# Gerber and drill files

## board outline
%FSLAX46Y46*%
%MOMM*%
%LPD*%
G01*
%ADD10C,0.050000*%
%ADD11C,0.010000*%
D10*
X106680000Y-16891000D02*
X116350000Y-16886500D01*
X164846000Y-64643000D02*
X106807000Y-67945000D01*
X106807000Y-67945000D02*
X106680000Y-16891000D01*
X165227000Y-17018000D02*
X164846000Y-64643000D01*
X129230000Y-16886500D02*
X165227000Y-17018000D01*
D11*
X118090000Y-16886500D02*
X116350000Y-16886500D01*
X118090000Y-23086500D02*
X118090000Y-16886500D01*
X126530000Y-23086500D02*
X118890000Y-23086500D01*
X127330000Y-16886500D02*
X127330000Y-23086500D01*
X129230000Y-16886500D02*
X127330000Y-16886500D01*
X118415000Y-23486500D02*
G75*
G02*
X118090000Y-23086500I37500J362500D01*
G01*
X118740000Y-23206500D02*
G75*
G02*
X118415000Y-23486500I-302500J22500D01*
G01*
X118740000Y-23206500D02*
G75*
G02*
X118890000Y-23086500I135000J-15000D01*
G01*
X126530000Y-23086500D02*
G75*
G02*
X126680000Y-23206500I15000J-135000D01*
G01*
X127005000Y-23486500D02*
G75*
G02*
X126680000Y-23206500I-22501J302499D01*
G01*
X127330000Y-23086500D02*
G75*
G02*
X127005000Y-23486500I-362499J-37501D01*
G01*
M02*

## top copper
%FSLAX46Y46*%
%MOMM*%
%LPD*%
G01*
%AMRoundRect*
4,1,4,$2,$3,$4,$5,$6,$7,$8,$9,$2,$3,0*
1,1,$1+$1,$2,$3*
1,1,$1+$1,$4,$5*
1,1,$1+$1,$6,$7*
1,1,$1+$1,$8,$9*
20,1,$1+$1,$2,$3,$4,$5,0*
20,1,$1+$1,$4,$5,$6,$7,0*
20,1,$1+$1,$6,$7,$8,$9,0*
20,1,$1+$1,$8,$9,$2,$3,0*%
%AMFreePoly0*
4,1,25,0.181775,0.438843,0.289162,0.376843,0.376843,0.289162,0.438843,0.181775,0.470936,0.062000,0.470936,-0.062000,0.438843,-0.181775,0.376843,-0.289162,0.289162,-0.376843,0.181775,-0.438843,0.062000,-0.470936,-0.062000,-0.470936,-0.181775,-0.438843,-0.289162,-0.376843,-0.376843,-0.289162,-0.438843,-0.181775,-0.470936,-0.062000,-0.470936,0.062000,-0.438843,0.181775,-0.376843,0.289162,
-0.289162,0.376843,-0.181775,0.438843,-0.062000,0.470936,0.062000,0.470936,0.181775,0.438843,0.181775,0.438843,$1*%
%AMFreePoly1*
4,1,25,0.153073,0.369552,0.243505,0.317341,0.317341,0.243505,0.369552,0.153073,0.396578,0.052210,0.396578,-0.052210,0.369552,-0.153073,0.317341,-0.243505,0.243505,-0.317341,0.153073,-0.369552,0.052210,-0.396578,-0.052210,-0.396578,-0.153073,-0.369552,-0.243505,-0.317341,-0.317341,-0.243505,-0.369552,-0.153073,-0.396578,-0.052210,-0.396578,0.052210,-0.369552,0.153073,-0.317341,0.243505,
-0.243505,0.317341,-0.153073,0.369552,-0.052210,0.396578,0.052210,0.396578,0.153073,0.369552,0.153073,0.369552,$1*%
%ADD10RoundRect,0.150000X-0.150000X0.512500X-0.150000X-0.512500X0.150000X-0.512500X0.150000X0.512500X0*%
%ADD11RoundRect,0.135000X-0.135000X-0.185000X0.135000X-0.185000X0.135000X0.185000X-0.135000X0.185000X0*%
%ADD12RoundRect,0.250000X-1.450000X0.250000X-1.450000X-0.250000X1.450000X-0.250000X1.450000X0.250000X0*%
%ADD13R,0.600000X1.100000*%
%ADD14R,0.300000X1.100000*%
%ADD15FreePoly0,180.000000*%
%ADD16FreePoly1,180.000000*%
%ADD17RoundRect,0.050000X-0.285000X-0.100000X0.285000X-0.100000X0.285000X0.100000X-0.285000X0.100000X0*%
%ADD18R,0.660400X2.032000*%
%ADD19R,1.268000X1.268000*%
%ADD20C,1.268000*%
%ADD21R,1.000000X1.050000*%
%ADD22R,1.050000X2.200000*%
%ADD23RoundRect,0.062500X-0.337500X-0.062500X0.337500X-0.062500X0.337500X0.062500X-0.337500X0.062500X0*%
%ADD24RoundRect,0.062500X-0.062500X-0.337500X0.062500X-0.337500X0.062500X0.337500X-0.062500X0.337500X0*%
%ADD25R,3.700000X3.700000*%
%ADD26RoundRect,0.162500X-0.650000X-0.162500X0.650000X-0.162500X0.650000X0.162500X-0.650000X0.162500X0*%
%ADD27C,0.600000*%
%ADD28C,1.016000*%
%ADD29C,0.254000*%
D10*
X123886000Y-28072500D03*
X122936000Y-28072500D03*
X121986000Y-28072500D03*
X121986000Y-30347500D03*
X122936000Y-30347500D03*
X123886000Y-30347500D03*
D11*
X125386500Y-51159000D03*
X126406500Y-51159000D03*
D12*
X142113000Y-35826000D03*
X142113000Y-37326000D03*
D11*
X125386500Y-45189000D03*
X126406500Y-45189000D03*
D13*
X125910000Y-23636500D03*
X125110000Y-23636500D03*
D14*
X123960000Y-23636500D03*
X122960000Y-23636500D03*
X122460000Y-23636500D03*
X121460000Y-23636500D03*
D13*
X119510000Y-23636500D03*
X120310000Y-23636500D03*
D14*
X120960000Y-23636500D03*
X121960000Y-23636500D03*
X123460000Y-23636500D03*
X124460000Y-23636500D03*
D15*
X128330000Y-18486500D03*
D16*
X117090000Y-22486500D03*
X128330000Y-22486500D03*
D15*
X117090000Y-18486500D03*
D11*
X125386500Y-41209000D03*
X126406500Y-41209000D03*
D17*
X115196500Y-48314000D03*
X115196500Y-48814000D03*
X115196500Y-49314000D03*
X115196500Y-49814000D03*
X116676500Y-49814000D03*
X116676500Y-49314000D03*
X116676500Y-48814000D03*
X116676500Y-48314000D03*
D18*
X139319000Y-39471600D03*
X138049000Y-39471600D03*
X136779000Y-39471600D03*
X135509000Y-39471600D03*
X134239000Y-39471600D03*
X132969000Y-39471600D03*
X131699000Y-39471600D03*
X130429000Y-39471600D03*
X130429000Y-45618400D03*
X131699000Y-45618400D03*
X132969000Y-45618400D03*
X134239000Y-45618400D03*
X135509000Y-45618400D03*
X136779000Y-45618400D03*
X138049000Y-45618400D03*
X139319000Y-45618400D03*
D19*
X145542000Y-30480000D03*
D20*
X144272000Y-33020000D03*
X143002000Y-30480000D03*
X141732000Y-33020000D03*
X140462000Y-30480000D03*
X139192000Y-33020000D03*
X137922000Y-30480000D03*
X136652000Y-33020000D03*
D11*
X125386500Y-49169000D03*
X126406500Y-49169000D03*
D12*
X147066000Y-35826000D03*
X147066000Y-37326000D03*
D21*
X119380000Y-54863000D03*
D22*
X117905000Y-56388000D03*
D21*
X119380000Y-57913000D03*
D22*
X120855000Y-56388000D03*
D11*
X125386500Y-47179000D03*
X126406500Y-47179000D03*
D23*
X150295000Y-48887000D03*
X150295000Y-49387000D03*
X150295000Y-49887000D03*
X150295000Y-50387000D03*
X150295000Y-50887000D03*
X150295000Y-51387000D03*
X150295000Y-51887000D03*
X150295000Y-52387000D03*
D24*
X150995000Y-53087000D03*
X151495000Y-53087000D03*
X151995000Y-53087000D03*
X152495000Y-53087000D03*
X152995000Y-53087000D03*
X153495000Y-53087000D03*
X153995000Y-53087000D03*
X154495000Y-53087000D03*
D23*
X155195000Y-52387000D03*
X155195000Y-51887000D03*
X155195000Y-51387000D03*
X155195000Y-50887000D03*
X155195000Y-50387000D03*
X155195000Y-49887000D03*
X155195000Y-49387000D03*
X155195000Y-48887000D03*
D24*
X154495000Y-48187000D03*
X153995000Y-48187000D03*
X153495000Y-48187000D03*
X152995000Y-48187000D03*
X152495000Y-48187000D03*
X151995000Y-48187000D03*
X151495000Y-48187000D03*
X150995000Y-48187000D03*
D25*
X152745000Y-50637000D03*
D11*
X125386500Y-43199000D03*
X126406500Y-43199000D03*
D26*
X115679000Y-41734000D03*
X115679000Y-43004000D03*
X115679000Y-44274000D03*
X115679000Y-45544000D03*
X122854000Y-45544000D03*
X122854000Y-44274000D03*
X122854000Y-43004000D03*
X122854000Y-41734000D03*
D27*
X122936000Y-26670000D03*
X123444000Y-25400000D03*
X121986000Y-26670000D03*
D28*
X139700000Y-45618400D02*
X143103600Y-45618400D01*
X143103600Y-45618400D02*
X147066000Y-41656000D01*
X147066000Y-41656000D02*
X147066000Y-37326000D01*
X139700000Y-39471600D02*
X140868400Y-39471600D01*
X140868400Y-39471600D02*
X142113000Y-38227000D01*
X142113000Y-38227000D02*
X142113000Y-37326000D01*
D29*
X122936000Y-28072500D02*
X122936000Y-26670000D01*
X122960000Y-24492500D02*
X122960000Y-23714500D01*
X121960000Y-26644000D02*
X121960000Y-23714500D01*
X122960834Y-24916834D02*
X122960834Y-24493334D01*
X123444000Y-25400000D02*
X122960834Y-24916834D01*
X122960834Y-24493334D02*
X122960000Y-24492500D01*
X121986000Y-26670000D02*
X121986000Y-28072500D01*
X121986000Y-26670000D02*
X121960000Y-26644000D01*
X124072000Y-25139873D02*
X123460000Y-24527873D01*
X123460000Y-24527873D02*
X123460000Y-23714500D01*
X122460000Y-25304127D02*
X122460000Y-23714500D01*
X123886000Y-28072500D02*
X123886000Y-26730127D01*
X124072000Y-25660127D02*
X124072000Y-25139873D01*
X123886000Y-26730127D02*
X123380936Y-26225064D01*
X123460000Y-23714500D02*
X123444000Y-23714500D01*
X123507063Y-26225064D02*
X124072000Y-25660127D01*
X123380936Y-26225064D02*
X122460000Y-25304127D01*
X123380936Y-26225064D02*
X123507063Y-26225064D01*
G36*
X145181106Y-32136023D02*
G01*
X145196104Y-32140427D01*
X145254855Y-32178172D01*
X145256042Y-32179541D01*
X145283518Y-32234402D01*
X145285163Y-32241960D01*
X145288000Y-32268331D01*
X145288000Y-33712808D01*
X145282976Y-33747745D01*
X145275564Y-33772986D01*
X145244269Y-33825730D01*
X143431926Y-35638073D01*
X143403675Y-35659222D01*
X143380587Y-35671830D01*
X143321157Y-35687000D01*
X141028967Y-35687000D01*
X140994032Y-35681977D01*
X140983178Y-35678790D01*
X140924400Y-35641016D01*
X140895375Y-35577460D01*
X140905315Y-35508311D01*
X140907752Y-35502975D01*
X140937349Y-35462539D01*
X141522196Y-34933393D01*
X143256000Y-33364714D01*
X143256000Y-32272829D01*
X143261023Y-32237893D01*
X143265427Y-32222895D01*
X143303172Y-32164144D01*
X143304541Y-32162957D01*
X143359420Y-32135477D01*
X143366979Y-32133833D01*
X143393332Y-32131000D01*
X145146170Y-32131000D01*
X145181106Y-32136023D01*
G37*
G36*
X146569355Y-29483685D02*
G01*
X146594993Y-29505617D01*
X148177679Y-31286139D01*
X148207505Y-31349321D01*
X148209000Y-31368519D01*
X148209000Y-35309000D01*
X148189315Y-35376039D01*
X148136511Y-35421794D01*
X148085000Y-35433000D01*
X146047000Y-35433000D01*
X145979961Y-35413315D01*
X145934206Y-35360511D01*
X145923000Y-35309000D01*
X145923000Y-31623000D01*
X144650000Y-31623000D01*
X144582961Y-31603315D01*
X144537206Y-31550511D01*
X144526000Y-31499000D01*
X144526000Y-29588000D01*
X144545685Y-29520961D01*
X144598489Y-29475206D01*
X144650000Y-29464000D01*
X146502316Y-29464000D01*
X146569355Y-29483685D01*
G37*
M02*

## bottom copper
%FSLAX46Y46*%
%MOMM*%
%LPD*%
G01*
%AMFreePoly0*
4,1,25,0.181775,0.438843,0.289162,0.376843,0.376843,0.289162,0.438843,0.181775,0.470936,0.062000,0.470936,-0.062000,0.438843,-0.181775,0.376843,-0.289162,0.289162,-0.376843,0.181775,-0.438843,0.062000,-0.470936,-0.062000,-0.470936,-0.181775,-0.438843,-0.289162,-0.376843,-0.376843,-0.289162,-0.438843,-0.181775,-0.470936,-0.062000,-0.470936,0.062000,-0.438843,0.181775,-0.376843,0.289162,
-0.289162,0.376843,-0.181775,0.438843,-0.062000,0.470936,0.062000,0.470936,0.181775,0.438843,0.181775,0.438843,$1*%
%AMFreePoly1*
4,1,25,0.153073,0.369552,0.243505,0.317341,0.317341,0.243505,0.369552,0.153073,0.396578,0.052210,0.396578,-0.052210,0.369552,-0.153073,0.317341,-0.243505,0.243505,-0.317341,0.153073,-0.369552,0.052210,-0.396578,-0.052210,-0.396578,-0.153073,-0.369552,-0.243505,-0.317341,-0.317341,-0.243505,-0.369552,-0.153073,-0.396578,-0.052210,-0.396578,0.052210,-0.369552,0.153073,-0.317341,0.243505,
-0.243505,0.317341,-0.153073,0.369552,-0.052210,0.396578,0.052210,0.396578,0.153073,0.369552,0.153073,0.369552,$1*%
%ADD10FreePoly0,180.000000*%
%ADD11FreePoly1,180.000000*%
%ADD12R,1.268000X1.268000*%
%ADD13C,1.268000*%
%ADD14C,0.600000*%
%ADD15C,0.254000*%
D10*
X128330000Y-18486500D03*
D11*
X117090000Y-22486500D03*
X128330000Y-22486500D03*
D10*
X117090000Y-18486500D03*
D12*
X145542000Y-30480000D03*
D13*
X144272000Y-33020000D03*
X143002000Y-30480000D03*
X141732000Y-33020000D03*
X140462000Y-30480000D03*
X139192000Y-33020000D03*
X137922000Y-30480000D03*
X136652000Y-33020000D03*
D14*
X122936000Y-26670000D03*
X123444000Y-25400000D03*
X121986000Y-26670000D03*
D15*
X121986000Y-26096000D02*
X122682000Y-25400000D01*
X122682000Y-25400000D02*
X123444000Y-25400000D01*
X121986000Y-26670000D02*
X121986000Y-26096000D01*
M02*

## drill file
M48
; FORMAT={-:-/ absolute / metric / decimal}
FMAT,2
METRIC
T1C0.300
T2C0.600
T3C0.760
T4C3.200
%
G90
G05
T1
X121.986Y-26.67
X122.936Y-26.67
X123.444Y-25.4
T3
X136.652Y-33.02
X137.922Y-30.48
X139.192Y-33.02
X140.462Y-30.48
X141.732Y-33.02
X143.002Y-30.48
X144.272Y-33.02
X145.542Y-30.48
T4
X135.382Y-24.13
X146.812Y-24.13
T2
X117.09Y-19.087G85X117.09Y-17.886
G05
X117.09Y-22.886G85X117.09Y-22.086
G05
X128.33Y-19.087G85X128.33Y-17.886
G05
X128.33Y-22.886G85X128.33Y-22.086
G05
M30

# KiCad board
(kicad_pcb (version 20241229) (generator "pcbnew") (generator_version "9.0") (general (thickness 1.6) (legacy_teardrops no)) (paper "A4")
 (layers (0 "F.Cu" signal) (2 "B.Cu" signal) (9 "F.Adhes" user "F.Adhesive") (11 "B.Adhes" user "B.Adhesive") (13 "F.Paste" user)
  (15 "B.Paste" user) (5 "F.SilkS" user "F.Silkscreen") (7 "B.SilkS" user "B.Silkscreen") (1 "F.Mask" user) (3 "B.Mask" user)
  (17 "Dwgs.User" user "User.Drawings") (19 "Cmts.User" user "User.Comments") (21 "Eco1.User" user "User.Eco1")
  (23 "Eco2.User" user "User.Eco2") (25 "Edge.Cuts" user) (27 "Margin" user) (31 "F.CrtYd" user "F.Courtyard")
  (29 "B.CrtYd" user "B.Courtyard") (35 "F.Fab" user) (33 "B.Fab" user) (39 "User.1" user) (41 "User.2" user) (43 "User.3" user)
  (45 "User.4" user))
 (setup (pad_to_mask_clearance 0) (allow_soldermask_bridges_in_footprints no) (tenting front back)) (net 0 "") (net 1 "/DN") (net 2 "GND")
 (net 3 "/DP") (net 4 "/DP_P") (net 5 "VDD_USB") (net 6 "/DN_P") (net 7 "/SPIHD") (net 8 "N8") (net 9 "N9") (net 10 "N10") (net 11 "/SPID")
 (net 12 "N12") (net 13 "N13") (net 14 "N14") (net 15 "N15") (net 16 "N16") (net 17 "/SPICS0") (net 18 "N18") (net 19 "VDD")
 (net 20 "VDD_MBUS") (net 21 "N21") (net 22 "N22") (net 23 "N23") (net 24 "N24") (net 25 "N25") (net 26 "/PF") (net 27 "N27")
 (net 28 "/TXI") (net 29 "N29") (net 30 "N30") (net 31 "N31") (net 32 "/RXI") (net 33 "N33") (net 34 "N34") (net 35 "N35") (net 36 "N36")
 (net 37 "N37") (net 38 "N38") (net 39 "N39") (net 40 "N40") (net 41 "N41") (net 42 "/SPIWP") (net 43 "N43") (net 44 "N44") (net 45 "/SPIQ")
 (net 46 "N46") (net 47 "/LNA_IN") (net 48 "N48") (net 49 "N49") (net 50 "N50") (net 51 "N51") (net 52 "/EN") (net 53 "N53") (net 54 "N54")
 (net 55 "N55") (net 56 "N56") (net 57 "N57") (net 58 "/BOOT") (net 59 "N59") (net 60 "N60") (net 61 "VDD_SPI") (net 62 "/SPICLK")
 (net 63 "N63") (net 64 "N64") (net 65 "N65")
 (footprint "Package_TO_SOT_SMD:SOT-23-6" (layer "F.Cu") (at 122.936 29.21 -90)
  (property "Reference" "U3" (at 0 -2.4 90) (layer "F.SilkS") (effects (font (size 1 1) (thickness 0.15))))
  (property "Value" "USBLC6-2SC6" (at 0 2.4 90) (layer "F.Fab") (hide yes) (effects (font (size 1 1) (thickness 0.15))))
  (pad "1" smd roundrect (at -1.1375 -0.95 270) (size 1.325 0.6) (layers "F.Cu" "F.Mask" "F.Paste") (roundrect_rratio 0.25) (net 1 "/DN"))
  (pad "2" smd roundrect (at -1.1375 0 270) (size 1.325 0.6) (layers "F.Cu" "F.Mask" "F.Paste") (roundrect_rratio 0.25) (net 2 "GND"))
  (pad "3" smd roundrect (at -1.1375 0.95 270) (size 1.325 0.6) (layers "F.Cu" "F.Mask" "F.Paste") (roundrect_rratio 0.25) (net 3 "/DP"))
  (pad "4" smd roundrect (at 1.1375 0.95 270) (size 1.325 0.6) (layers "F.Cu" "F.Mask" "F.Paste") (roundrect_rratio 0.25) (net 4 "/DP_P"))
  (pad "5" smd roundrect (at 1.1375 0 270) (size 1.325 0.6) (layers "F.Cu" "F.Mask" "F.Paste") (roundrect_rratio 0.25) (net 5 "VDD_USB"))
  (pad "6" smd roundrect (at 1.1375 -0.95 270) (size 1.325 0.6) (layers "F.Cu" "F.Mask" "F.Paste") (roundrect_rratio 0.25) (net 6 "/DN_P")))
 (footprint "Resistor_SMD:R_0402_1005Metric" (layer "F.Cu") (at 125.8965 51.159)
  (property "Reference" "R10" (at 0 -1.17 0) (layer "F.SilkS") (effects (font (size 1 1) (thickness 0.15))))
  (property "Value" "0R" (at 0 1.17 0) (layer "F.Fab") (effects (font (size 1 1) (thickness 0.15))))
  (pad "1" smd roundrect (at -0.51 0) (size 0.54 0.64) (layers "F.Cu" "F.Mask" "F.Paste") (roundrect_rratio 0.25) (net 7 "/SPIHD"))
  (pad "2" smd roundrect (at 0.51 0) (size 0.54 0.64) (layers "F.Cu" "F.Mask" "F.Paste") (roundrect_rratio 0.25) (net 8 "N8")))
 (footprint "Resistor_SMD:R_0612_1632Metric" (layer "F.Cu") (at 142.113 36.576 -90)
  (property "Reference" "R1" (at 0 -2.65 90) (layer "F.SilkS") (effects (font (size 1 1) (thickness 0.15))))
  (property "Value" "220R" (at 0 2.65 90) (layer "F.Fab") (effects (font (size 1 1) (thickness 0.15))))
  (pad "1" smd roundrect (at -0.75 0 270) (size 1 3.4) (layers "F.Cu" "F.Mask" "F.Paste") (roundrect_rratio 0.25) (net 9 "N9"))
  (pad "2" smd roundrect (at 0.75 0 270) (size 1 3.4) (layers "F.Cu" "F.Mask" "F.Paste") (roundrect_rratio 0.25) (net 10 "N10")))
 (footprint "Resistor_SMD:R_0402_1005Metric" (layer "F.Cu") (at 125.8965 45.189)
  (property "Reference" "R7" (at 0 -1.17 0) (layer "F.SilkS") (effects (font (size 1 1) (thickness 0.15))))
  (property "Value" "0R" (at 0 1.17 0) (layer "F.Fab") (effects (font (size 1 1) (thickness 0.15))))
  (pad "1" smd roundrect (at -0.51 0) (size 0.54 0.64) (layers "F.Cu" "F.Mask" "F.Paste") (roundrect_rratio 0.25) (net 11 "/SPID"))
  (pad "2" smd roundrect (at 0.51 0) (size 0.54 0.64) (layers "F.Cu" "F.Mask" "F.Paste") (roundrect_rratio 0.25) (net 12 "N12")))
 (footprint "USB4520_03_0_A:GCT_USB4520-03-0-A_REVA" (layer "F.Cu") (at 122.71 18.4865 180)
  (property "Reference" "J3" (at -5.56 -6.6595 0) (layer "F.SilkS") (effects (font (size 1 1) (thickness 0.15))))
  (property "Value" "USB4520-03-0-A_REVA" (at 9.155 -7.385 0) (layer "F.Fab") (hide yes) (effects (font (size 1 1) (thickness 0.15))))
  (fp_line (start 4.62 1.6) (end 6.36 1.6) (stroke (width 0.01) (type solid)) (layer "Edge.Cuts"))
  (fp_line (start 4.62 -4.6) (end 4.62 1.6) (stroke (width 0.01) (type solid)) (layer "Edge.Cuts"))
  (fp_line (start -3.82 -4.6) (end 3.82 -4.6) (stroke (width 0.01) (type solid)) (layer "Edge.Cuts"))
  (fp_line (start -4.62 1.6) (end -4.62 -4.6) (stroke (width 0.01) (type solid)) (layer "Edge.Cuts"))
  (fp_line (start -6.52 1.6) (end -4.62 1.6) (stroke (width 0.01) (type solid)) (layer "Edge.Cuts"))
  (fp_arc (start 4.295 -5) (mid 4.540343 -4.86731) (end 4.62 -4.6) (stroke (width 0.01) (type solid)) (layer "Edge.Cuts"))
  (fp_arc (start 3.97 -4.72) (mid 4.07451 -4.92731) (end 4.295 -5) (stroke (width 0.01) (type solid)) (layer "Edge.Cuts"))
  (fp_arc (start 3.97 -4.72) (mid 3.919853 -4.628934) (end 3.82 -4.6) (stroke (width 0.01) (type solid)) (layer "Edge.Cuts"))
  (fp_arc (start -3.82 -4.6) (mid -3.919853 -4.628934) (end -3.97 -4.72) (stroke (width 0.01) (type solid)) (layer "Edge.Cuts"))
  (fp_arc (start -4.295 -5) (mid -4.07451 -4.92731) (end -3.97 -4.72) (stroke (width 0.01) (type solid)) (layer "Edge.Cuts"))
  (fp_arc (start -4.62 -4.6) (mid -4.540343 -4.86731) (end -4.295 -5) (stroke (width 0.01) (type solid)) (layer "Edge.Cuts"))
  (pad "A1_B12" smd rect (at -3.2 -5.15 180) (size 0.6 1.1) (layers "F.Cu" "F.Mask" "F.Paste") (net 2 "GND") (solder_mask_margin 0.102))
  (pad "A4_B9" smd rect (at -2.4 -5.15 180) (size 0.6 1.1) (layers "F.Cu" "F.Mask" "F.Paste") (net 5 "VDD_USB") (solder_mask_margin 0.102))
  (pad "A5" smd rect (at -1.25 -5.15 180) (size 0.3 1.1) (layers "F.Cu" "F.Mask" "F.Paste") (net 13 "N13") (solder_mask_margin 0.102))
  (pad "A6" smd rect (at -0.25 -5.15 180) (size 0.3 1.1) (layers "F.Cu" "F.Mask" "F.Paste") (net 3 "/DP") (solder_mask_margin 0.102))
  (pad "A7" smd rect (at 0.25 -5.15 180) (size 0.3 1.1) (layers "F.Cu" "F.Mask" "F.Paste") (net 1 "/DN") (solder_mask_margin 0.102))
  (pad "A8" smd rect (at 1.25 -5.15 180) (size 0.3 1.1) (layers "F.Cu" "F.Mask" "F.Paste") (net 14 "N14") (solder_mask_margin 0.102))
  (pad "B1_A12" smd rect (at 3.2 -5.15 180) (size 0.6 1.1) (layers "F.Cu" "F.Mask" "F.Paste") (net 2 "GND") (solder_mask_margin 0.102))
  (pad "B4_A9" smd rect (at 2.4 -5.15 180) (size 0.6 1.1) (layers "F.Cu" "F.Mask" "F.Paste") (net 5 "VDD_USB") (solder_mask_margin 0.102))
  (pad "B5" smd rect (at 1.75 -5.15 180) (size 0.3 1.1) (layers "F.Cu" "F.Mask" "F.Paste") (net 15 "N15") (solder_mask_margin 0.102))
  (pad "B6" smd rect (at 0.75 -5.15 180) (size 0.3 1.1) (layers "F.Cu" "F.Mask" "F.Paste") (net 3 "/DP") (solder_mask_margin 0.102))
  (pad "B7" smd rect (at -0.75 -5.15 180) (size 0.3 1.1) (layers "F.Cu" "F.Mask" "F.Paste") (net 1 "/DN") (solder_mask_margin 0.102))
  (pad "B8" smd rect (at -1.75 -5.15 180) (size 0.3 1.1) (layers "F.Cu" "F.Mask" "F.Paste") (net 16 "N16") (solder_mask_margin 0.102))
  (pad "S1" thru_hole custom (at -5.62 0 180) (size 0.95 1.9) (drill oval 0.6 1.8) (layers "*.Cu") (remove_unused_layers no) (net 2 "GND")
   (thermal_bridge_angle 90) (options (clearance outline) (anchor circle)) (primitives))
  (pad "S2" thru_hole custom (at 5.62 -4 180) (size 0.8 1.6) (drill oval 0.6 1.4) (layers "*.Cu") (remove_unused_layers no) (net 2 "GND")
   (thermal_bridge_angle 90) (options (clearance outline) (anchor circle)) (primitives))
  (pad "S3" thru_hole custom (at -5.62 -4 180) (size 0.8 1.6) (drill oval 0.6 1.4) (layers "*.Cu") (remove_unused_layers no) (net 2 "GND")
   (thermal_bridge_angle 90) (options (clearance outline) (anchor circle)) (primitives))
  (pad "S4" thru_hole custom (at 5.62 0 180) (size 0.95 1.9) (drill oval 0.6 1.8) (layers "*.Cu") (remove_unused_layers no) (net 2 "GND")
   (thermal_bridge_angle 90) (options (clearance outline) (anchor circle)) (primitives)))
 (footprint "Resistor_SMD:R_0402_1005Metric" (layer "F.Cu") (at 125.8965 41.209)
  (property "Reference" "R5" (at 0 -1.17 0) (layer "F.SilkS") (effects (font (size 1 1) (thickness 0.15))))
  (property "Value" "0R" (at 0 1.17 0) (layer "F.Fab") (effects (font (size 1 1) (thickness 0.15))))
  (pad "1" smd roundrect (at -0.51 0) (size 0.54 0.64) (layers "F.Cu" "F.Mask" "F.Paste") (roundrect_rratio 0.25) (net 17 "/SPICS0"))
  (pad "2" smd roundrect (at 0.51 0) (size 0.54 0.64) (layers "F.Cu" "F.Mask" "F.Paste") (roundrect_rratio 0.25) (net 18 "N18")))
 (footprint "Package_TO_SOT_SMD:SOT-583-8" (layer "F.Cu") (at 115.9365 49.064)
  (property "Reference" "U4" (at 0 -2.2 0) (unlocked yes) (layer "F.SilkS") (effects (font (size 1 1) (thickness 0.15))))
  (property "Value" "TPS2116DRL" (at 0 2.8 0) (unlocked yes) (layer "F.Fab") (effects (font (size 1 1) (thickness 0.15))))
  (pad "1" smd roundrect (at -0.74 -0.75) (size 0.67 0.3) (layers "F.Cu" "F.Mask" "F.Paste") (roundrect_rratio 0.1666666667) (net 2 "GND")
   (thermal_bridge_angle 45))
  (pad "2" smd roundrect (at -0.74 -0.25) (size 0.67 0.3) (layers "F.Cu" "F.Mask" "F.Paste") (roundrect_rratio 0.1666666667) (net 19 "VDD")
   (thermal_bridge_angle 45))
  (pad "3" smd roundrect (at -0.74 0.25) (size 0.67 0.3) (layers "F.Cu" "F.Mask" "F.Paste") (roundrect_rratio 0.1666666667)
   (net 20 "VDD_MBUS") (thermal_bridge_angle 45))
  (pad "4" smd roundrect (at -0.74 0.75) (size 0.67 0.3) (layers "F.Cu" "F.Mask" "F.Paste") (roundrect_rratio 0.1666666667) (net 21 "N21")
   (thermal_bridge_angle 45))
  (pad "5" smd roundrect (at 0.74 0.75) (size 0.67 0.3) (layers "F.Cu" "F.Mask" "F.Paste") (roundrect_rratio 0.1666666667)
   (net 20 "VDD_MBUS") (thermal_bridge_angle 45))
  (pad "6" smd roundrect (at 0.74 0.25) (size 0.67 0.3) (layers "F.Cu" "F.Mask" "F.Paste") (roundrect_rratio 0.1666666667) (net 5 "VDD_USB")
   (thermal_bridge_angle 45))
  (pad "7" smd roundrect (at 0.74 -0.25) (size 0.67 0.3) (layers "F.Cu" "F.Mask" "F.Paste") (roundrect_rratio 0.1666666667) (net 19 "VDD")
   (thermal_bridge_angle 45))
  (pad "8" smd roundrect (at 0.74 -0.75) (size 0.67 0.3) (layers "F.Cu" "F.Mask" "F.Paste") (roundrect_rratio 0.1666666667) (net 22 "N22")
   (thermal_bridge_angle 45)))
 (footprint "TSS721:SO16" (layer "F.Cu") (at 134.874 42.545 180)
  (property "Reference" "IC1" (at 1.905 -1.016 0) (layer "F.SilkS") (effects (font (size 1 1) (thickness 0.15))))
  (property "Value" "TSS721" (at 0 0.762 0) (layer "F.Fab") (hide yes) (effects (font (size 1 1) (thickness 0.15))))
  (pad "1" smd rect (at -4.445 3.0734 180) (size 0.6604 2.032) (layers "F.Cu" "F.Mask" "F.Paste") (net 10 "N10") (solder_mask_margin 0.102))
  (pad "2" smd rect (at -3.175 3.0734 180) (size 0.6604 2.032) (layers "F.Cu" "F.Mask" "F.Paste") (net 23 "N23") (solder_mask_margin 0.102))
  (pad "3" smd rect (at -1.905 3.0734 180) (size 0.6604 2.032) (layers "F.Cu" "F.Mask" "F.Paste") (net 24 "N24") (solder_mask_margin 0.102))
  (pad "4" smd rect (at -0.635 3.0734 180) (size 0.6604 2.032) (layers "F.Cu" "F.Mask" "F.Paste") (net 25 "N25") (solder_mask_margin 0.102))
  (pad "5" smd rect (at 0.635 3.0734 180) (size 0.6604 2.032) (layers "F.Cu" "F.Mask" "F.Paste") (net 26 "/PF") (solder_mask_margin 0.102))
  (pad "6" smd rect (at 1.905 3.0734 180) (size 0.6604 2.032) (layers "F.Cu" "F.Mask" "F.Paste") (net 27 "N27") (solder_mask_margin 0.102))
  (pad "7" smd rect (at 3.175 3.0734 180) (size 0.6604 2.032) (layers "F.Cu" "F.Mask" "F.Paste") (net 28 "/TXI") (solder_mask_margin 0.102))
  (pad "8" smd rect (at 4.445 3.0734 180) (size 0.6604 2.032) (layers "F.Cu" "F.Mask" "F.Paste") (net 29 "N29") (solder_mask_margin 0.102))
  (pad "9" smd rect (at 4.445 -3.0734 180) (size 0.6604 2.032) (layers "F.Cu" "F.Mask" "F.Paste") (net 20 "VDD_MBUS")
   (solder_mask_margin 0.102))
  (pad "10" smd rect (at 3.175 -3.0734 180) (size 0.6604 2.032) (layers "F.Cu" "F.Mask" "F.Paste") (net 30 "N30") (solder_mask_margin 0.102))
  (pad "11" smd rect (at 1.905 -3.0734 180) (size 0.6604 2.032) (layers "F.Cu" "F.Mask" "F.Paste") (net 20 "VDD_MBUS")
   (solder_mask_margin 0.102))
  (pad "12" smd rect (at 0.635 -3.0734 180) (size 0.6604 2.032) (layers "F.Cu" "F.Mask" "F.Paste") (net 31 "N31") (solder_mask_margin 0.102))
  (pad "13" smd rect (at -0.635 -3.0734 180) (size 0.6604 2.032) (layers "F.Cu" "F.Mask" "F.Paste") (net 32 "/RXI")
   (solder_mask_margin 0.102))
  (pad "14" smd rect (at -1.905 -3.0734 180) (size 0.6604 2.032) (layers "F.Cu" "F.Mask" "F.Paste") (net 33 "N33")
   (solder_mask_margin 0.102))
  (pad "15" smd rect (at -3.175 -3.0734 180) (size 0.6604 2.032) (layers "F.Cu" "F.Mask" "F.Paste") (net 2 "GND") (solder_mask_margin 0.102))
  (pad "16" smd rect (at -4.445 -3.0734 180) (size 0.6604 2.032) (layers "F.Cu" "F.Mask" "F.Paste") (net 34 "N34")
   (solder_mask_margin 0.102)))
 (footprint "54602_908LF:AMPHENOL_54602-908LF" (layer "F.Cu") (at 141.097 24.13 180)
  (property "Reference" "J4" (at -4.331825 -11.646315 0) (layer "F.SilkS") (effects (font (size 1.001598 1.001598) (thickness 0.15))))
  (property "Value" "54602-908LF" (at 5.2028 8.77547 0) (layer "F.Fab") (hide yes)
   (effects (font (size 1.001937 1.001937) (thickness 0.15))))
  (pad "" np_thru_hole circle (at -5.715 0 180) (size 3.2 3.2) (drill 3.2) (layers "*.Cu" "*.Mask"))
  (pad "" np_thru_hole circle (at 5.715 0 180) (size 3.2 3.2) (drill 3.2) (layers "*.Cu" "*.Mask"))
  (pad "1" thru_hole rect (at -4.445 -6.35 180) (size 1.268 1.268) (drill 0.76) (layers "*.Cu" "*.Mask") (remove_unused_layers no)
   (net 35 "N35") (solder_mask_margin 0.102))
  (pad "2" thru_hole circle (at -3.175 -8.89 180) (size 1.268 1.268) (drill 0.76) (layers "*.Cu" "*.Mask") (remove_unused_layers no)
   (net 9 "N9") (solder_mask_margin 0.102))
  (pad "3" thru_hole circle (at -1.905 -6.35 180) (size 1.268 1.268) (drill 0.76) (layers "*.Cu" "*.Mask") (remove_unused_layers no)
   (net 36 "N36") (solder_mask_margin 0.102))
  (pad "4" thru_hole circle (at -0.635 -8.89 180) (size 1.268 1.268) (drill 0.76) (layers "*.Cu" "*.Mask") (remove_unused_layers no)
   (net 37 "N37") (solder_mask_margin 0.102))
  (pad "5" thru_hole circle (at 0.635 -6.35 180) (size 1.268 1.268) (drill 0.76) (layers "*.Cu" "*.Mask") (remove_unused_layers no)
   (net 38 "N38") (solder_mask_margin 0.102))
  (pad "6" thru_hole circle (at 1.905 -8.89 180) (size 1.268 1.268) (drill 0.76) (layers "*.Cu" "*.Mask") (remove_unused_layers no)
   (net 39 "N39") (solder_mask_margin 0.102))
  (pad "7" thru_hole circle (at 3.175 -6.35 180) (size 1.268 1.268) (drill 0.76) (layers "*.Cu" "*.Mask") (remove_unused_layers no)
   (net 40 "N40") (solder_mask_margin 0.102))
  (pad "8" thru_hole circle (at 4.445 -8.89 180) (size 1.268 1.268) (drill 0.76) (layers "*.Cu" "*.Mask") (remove_unused_layers no)
   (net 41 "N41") (solder_mask_margin 0.102)))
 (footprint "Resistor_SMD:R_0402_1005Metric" (layer "F.Cu") (at 125.8965 49.169)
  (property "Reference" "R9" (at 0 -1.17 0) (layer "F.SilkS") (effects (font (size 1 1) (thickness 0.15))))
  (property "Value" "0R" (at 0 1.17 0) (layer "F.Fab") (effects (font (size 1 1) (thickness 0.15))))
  (pad "1" smd roundrect (at -0.51 0) (size 0.54 0.64) (layers "F.Cu" "F.Mask" "F.Paste") (roundrect_rratio 0.25) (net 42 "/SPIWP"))
  (pad "2" smd roundrect (at 0.51 0) (size 0.54 0.64) (layers "F.Cu" "F.Mask" "F.Paste") (roundrect_rratio 0.25) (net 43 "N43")))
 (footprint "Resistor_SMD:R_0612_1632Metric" (layer "F.Cu") (at 147.066 36.576 -90)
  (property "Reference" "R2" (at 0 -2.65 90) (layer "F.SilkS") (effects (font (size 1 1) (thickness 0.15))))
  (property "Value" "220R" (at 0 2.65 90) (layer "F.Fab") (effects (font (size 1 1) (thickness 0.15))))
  (pad "1" smd roundrect (at -0.75 0 270) (size 1 3.4) (layers "F.Cu" "F.Mask" "F.Paste") (roundrect_rratio 0.25) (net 35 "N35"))
  (pad "2" smd roundrect (at 0.75 0 270) (size 1 3.4) (layers "F.Cu" "F.Mask" "F.Paste") (roundrect_rratio 0.25) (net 34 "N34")))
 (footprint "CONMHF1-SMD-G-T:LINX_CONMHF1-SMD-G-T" (layer "F.Cu") (at 119.38 56.388)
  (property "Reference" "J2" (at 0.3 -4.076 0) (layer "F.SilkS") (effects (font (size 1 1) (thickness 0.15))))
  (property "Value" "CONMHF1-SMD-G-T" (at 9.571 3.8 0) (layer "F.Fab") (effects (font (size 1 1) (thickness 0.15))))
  (pad "1" smd rect (at 0 -1.525) (size 1 1.05) (layers "F.Cu" "F.Mask" "F.Paste") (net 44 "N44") (solder_mask_margin 0.102))
  (pad "S1" smd rect (at -1.475 0) (size 1.05 2.2) (layers "F.Cu" "F.Mask" "F.Paste") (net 2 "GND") (solder_mask_margin 0.102))
  (pad "S2" smd rect (at 0 1.525) (size 1 1.05) (layers "F.Cu" "F.Mask" "F.Paste") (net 2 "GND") (solder_mask_margin 0.102))
  (pad "S3" smd rect (at 1.475 0) (size 1.05 2.2) (layers "F.Cu" "F.Mask" "F.Paste") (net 2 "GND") (solder_mask_margin 0.102))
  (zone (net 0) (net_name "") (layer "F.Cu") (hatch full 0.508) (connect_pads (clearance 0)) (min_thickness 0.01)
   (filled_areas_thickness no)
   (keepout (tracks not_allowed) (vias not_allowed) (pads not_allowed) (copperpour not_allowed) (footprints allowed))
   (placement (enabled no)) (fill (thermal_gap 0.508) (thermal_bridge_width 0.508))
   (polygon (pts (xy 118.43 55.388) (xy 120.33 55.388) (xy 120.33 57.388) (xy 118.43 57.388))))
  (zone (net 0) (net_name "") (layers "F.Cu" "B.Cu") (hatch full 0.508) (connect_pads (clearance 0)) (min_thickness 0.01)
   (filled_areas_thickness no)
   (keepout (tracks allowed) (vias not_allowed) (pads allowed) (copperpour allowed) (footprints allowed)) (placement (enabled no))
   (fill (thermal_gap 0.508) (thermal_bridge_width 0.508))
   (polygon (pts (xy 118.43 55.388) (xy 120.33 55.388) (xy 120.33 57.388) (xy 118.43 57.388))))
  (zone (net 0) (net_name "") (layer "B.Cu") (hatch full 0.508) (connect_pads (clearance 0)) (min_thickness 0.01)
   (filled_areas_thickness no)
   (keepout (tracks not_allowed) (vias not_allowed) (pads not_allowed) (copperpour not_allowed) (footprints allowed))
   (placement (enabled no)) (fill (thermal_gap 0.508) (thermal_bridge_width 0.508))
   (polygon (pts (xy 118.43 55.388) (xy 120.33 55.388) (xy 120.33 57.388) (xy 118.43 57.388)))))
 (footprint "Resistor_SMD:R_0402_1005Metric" (layer "F.Cu") (at 125.8965 47.179)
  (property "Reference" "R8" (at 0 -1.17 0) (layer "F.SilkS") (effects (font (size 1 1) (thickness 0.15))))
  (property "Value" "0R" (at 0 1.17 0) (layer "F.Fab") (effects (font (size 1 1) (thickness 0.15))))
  (pad "1" smd roundrect (at -0.51 0) (size 0.54 0.64) (layers "F.Cu" "F.Mask" "F.Paste") (roundrect_rratio 0.25) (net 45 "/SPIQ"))
  (pad "2" smd roundrect (at 0.51 0) (size 0.54 0.64) (layers "F.Cu" "F.Mask" "F.Paste") (roundrect_rratio 0.25) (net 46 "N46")))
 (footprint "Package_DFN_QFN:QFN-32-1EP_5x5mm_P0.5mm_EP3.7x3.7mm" (layer "F.Cu") (at 152.745 50.637)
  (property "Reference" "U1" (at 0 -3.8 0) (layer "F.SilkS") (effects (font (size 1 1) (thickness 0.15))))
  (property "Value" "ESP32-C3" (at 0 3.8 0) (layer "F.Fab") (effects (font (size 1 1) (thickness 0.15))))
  (pad "" smd roundrect (at -0.925 -0.925) (size 1.49 1.49) (layers "F.Paste") (roundrect_rratio 0.167785))
  (pad "" smd roundrect (at -0.925 0.925) (size 1.49 1.49) (layers "F.Paste") (roundrect_rratio 0.167785))
  (pad "" smd roundrect (at 0.925 -0.925) (size 1.49 1.49) (layers "F.Paste") (roundrect_rratio 0.167785))
  (pad "" smd roundrect (at 0.925 0.925) (size 1.49 1.49) (layers "F.Paste") (roundrect_rratio 0.167785))
  (pad "1" smd roundrect (at -2.45 -1.75) (size 0.8 0.25) (layers "F.Cu" "F.Mask" "F.Paste") (roundrect_rratio 0.25) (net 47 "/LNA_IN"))
  (pad "2" smd roundrect (at -2.45 -1.25) (size 0.8 0.25) (layers "F.Cu" "F.Mask" "F.Paste") (roundrect_rratio 0.25) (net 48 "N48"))
  (pad "3" smd roundrect (at -2.45 -0.75) (size 0.8 0.25) (layers "F.Cu" "F.Mask" "F.Paste") (roundrect_rratio 0.25) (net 48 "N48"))
  (pad "4" smd roundrect (at -2.45 -0.25) (size 0.8 0.25) (layers "F.Cu" "F.Mask" "F.Paste") (roundrect_rratio 0.25) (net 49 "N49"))
  (pad "5" smd roundrect (at -2.45 0.25) (size 0.8 0.25) (layers "F.Cu" "F.Mask" "F.Paste") (roundrect_rratio 0.25) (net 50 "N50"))
  (pad "6" smd roundrect (at -2.45 0.75) (size 0.8 0.25) (layers "F.Cu" "F.Mask" "F.Paste") (roundrect_rratio 0.25) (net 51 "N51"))
  (pad "7" smd roundrect (at -2.45 1.25) (size 0.8 0.25) (layers "F.Cu" "F.Mask" "F.Paste") (roundrect_rratio 0.25) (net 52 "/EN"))
  (pad "8" smd roundrect (at -2.45 1.75) (size 0.8 0.25) (layers "F.Cu" "F.Mask" "F.Paste") (roundrect_rratio 0.25) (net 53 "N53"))
  (pad "9" smd roundrect (at -1.75 2.45) (size 0.25 0.8) (layers "F.Cu" "F.Mask" "F.Paste") (roundrect_rratio 0.25) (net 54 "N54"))
  (pad "10" smd roundrect (at -1.25 2.45) (size 0.25 0.8) (layers "F.Cu" "F.Mask" "F.Paste") (roundrect_rratio 0.25) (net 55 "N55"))
  (pad "11" smd roundrect (at -0.75 2.45) (size 0.25 0.8) (layers "F.Cu" "F.Mask" "F.Paste") (roundrect_rratio 0.25) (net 19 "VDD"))
  (pad "12" smd roundrect (at -0.25 2.45) (size 0.25 0.8) (layers "F.Cu" "F.Mask" "F.Paste") (roundrect_rratio 0.25) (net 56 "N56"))
  (pad "13" smd roundrect (at 0.25 2.45) (size 0.25 0.8) (layers "F.Cu" "F.Mask" "F.Paste") (roundrect_rratio 0.25) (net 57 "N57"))
  (pad "14" smd roundrect (at 0.75 2.45) (size 0.25 0.8) (layers "F.Cu" "F.Mask" "F.Paste") (roundrect_rratio 0.25) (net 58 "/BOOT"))
  (pad "15" smd roundrect (at 1.25 2.45) (size 0.25 0.8) (layers "F.Cu" "F.Mask" "F.Paste") (roundrect_rratio 0.25) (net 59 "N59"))
  (pad "16" smd roundrect (at 1.75 2.45) (size 0.25 0.8) (layers "F.Cu" "F.Mask" "F.Paste") (roundrect_rratio 0.25) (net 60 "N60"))
  (pad "17" smd roundrect (at 2.45 1.75) (size 0.8 0.25) (layers "F.Cu" "F.Mask" "F.Paste") (roundrect_rratio 0.25) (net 19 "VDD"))
  (pad "18" smd roundrect (at 2.45 1.25) (size 0.8 0.25) (layers "F.Cu" "F.Mask" "F.Paste") (roundrect_rratio 0.25) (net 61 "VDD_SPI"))
  (pad "19" smd roundrect (at 2.45 0.75) (size 0.8 0.25) (layers "F.Cu" "F.Mask" "F.Paste") (roundrect_rratio 0.25) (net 7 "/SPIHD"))
  (pad "20" smd roundrect (at 2.45 0.25) (size 0.8 0.25) (layers "F.Cu" "F.Mask" "F.Paste") (roundrect_rratio 0.25) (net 42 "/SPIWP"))
  (pad "21" smd roundrect (at 2.45 -0.25) (size 0.8 0.25) (layers "F.Cu" "F.Mask" "F.Paste") (roundrect_rratio 0.25) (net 17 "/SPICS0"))
  (pad "22" smd roundrect (at 2.45 -0.75) (size 0.8 0.25) (layers "F.Cu" "F.Mask" "F.Paste") (roundrect_rratio 0.25) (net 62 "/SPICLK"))
  (pad "23" smd roundrect (at 2.45 -1.25) (size 0.8 0.25) (layers "F.Cu" "F.Mask" "F.Paste") (roundrect_rratio 0.25) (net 11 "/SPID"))
  (pad "24" smd roundrect (at 2.45 -1.75) (size 0.8 0.25) (layers "F.Cu" "F.Mask" "F.Paste") (roundrect_rratio 0.25) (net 45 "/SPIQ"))
  (pad "25" smd roundrect (at 1.75 -2.45) (size 0.25 0.8) (layers "F.Cu" "F.Mask" "F.Paste") (roundrect_rratio 0.25) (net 6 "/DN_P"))
  (pad "26" smd roundrect (at 1.25 -2.45) (size 0.25 0.8) (layers "F.Cu" "F.Mask" "F.Paste") (roundrect_rratio 0.25) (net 4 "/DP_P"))
  (pad "27" smd roundrect (at 0.75 -2.45) (size 0.25 0.8) (layers "F.Cu" "F.Mask" "F.Paste") (roundrect_rratio 0.25) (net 28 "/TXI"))
  (pad "28" smd roundrect (at 0.25 -2.45) (size 0.25 0.8) (layers "F.Cu" "F.Mask" "F.Paste") (roundrect_rratio 0.25) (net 32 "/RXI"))
  (pad "29" smd roundrect (at -0.25 -2.45) (size 0.25 0.8) (layers "F.Cu" "F.Mask" "F.Paste") (roundrect_rratio 0.25) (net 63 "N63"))
  (pad "30" smd roundrect (at -0.75 -2.45) (size 0.25 0.8) (layers "F.Cu" "F.Mask" "F.Paste") (roundrect_rratio 0.25) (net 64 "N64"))
  (pad "31" smd roundrect (at -1.25 -2.45) (size 0.25 0.8) (layers "F.Cu" "F.Mask" "F.Paste") (roundrect_rratio 0.25) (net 19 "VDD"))
  (pad "32" smd roundrect (at -1.75 -2.45) (size 0.25 0.8) (layers "F.Cu" "F.Mask" "F.Paste") (roundrect_rratio 0.25) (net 19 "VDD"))
  (pad "33" smd rect (at 0 0) (size 3.7 3.7) (layers "F.Cu" "F.Mask") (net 2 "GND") (zone_connect 2)))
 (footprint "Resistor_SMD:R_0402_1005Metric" (layer "F.Cu") (at 125.8965 43.199)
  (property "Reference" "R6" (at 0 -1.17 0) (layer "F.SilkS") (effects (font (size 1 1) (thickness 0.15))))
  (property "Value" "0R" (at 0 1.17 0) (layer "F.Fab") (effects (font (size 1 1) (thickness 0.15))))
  (pad "1" smd roundrect (at -0.51 0) (size 0.54 0.64) (layers "F.Cu" "F.Mask" "F.Paste") (roundrect_rratio 0.25) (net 62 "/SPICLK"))
  (pad "2" smd roundrect (at 0.51 0) (size 0.54 0.64) (layers "F.Cu" "F.Mask" "F.Paste") (roundrect_rratio 0.25) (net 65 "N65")))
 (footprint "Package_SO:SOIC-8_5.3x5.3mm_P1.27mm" (layer "F.Cu") (at 119.2665 43.639)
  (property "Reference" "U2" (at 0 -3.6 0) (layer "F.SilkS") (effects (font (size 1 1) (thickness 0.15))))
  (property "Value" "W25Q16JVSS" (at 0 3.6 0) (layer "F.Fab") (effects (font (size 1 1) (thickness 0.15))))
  (pad "1" smd roundrect (at -3.5875 -1.905) (size 1.625 0.65) (layers "F.Cu" "F.Mask" "F.Paste") (roundrect_rratio 0.25) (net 18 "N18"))
  (pad "2" smd roundrect (at -3.5875 -0.635) (size 1.625 0.65) (layers "F.Cu" "F.Mask" "F.Paste") (roundrect_rratio 0.25) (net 46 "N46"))
  (pad "3" smd roundrect (at -3.5875 0.635) (size 1.625 0.65) (layers "F.Cu" "F.Mask" "F.Paste") (roundrect_rratio 0.25) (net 43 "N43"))
  (pad "4" smd roundrect (at -3.5875 1.905) (size 1.625 0.65) (layers "F.Cu" "F.Mask" "F.Paste") (roundrect_rratio 0.25) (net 2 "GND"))
  (pad "5" smd roundrect (at 3.5875 1.905) (size 1.625 0.65) (layers "F.Cu" "F.Mask" "F.Paste") (roundrect_rratio 0.25) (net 12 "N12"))
  (pad "6" smd roundrect (at 3.5875 0.635) (size 1.625 0.65) (layers "F.Cu" "F.Mask" "F.Paste") (roundrect_rratio 0.25) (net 65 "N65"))
  (pad "7" smd roundrect (at 3.5875 -0.635) (size 1.625 0.65) (layers "F.Cu" "F.Mask" "F.Paste") (roundrect_rratio 0.25) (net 8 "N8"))
  (pad "8" smd roundrect (at 3.5875 -1.905) (size 1.625 0.65) (layers "F.Cu" "F.Mask" "F.Paste") (roundrect_rratio 0.25) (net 61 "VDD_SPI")))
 (gr_line (start 106.68 16.891) (end 116.35 16.8865) (stroke (width 0.05) (type default)) (layer "Edge.Cuts"))
 (gr_line (start 164.846 64.643) (end 106.807 67.945) (stroke (width 0.05) (type default)) (layer "Edge.Cuts"))
 (gr_line (start 106.807 67.945) (end 106.68 16.891) (stroke (width 0.05) (type default)) (layer "Edge.Cuts"))
 (gr_line (start 165.227 17.018) (end 164.846 64.643) (stroke (width 0.05) (type default)) (layer "Edge.Cuts"))
 (gr_line (start 129.23 16.8865) (end 165.227 17.018) (stroke (width 0.05) (type default)) (layer "Edge.Cuts"))
 (segment (start 139.7 45.6184) (end 143.1036 45.6184) (width 1.016) (layer "F.Cu") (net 34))
 (segment (start 143.1036 45.6184) (end 147.066 41.656) (width 1.016) (layer "F.Cu") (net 34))
 (segment (start 147.066 41.656) (end 147.066 37.326) (width 1.016) (layer "F.Cu") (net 34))
 (segment (start 139.7 39.4716) (end 140.8684 39.4716) (width 1.016) (layer "F.Cu") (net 10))
 (segment (start 140.8684 39.4716) (end 142.113 38.227) (width 1.016) (layer "F.Cu") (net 10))
 (segment (start 142.113 38.227) (end 142.113 37.326) (width 1.016) (layer "F.Cu") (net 10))
 (segment (start 122.936 28.0725) (end 122.936 26.67) (width 0.254) (layer "F.Cu") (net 2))
 (via (at 122.936 26.67) (size 0.6) (drill 0.3) (layers "F.Cu" "B.Cu") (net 2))
 (segment (start 122.96 24.4925) (end 122.96 23.7145) (width 0.254) (layer "F.Cu") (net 3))
 (segment (start 121.96 26.644) (end 121.96 23.7145) (width 0.254) (layer "F.Cu") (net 3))
 (segment (start 122.960834 24.916834) (end 122.960834 24.493334) (width 0.254) (layer "F.Cu") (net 3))
 (segment (start 123.444 25.4) (end 122.960834 24.916834) (width 0.254) (layer "F.Cu") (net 3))
 (segment (start 122.960834 24.493334) (end 122.96 24.4925) (width 0.254) (layer "F.Cu") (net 3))
 (segment (start 121.986 26.67) (end 121.986 28.0725) (width 0.254) (layer "F.Cu") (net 3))
 (segment (start 121.986 26.67) (end 121.96 26.644) (width 0.254) (layer "F.Cu") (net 3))
 (via (at 123.444 25.4) (size 0.6) (drill 0.3) (layers "F.Cu" "B.Cu") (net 3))
 (via (at 121.986 26.67) (size 0.6) (drill 0.3) (layers "F.Cu" "B.Cu") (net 3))
 (segment (start 121.986 26.096) (end 122.682 25.4) (width 0.254) (layer "B.Cu") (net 3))
 (segment (start 122.682 25.4) (end 123.444 25.4) (width 0.254) (layer "B.Cu") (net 3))
 (segment (start 121.986 26.67) (end 121.986 26.096) (width 0.254) (layer "B.Cu") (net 3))
 (segment (start 124.072 25.139873) (end 123.46 24.527873) (width 0.254) (layer "F.Cu") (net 1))
 (segment (start 123.46 24.527873) (end 123.46 23.7145) (width 0.254) (layer "F.Cu") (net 1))
 (segment (start 122.46 25.304127) (end 122.46 23.7145) (width 0.254) (layer "F.Cu") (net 1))
 (segment (start 123.886 28.0725) (end 123.886 26.730127) (width 0.254) (layer "F.Cu") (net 1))
 (segment (start 124.072 25.660127) (end 124.072 25.139873) (width 0.254) (layer "F.Cu") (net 1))
 (segment (start 123.886 26.730127) (end 123.380936 26.225064) (width 0.254) (layer "F.Cu") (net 1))
 (segment (start 123.46 23.7145) (end 123.444 23.7145) (width 0.254) (layer "F.Cu") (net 1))
 (segment (start 123.507063 26.225064) (end 124.072 25.660127) (width 0.254) (layer "F.Cu") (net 1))
 (segment (start 123.380936 26.225064) (end 122.46 25.304127) (width 0.254) (layer "F.Cu") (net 1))
 (segment (start 123.380936 26.225064) (end 123.507063 26.225064) (width 0.254) (layer "F.Cu") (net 1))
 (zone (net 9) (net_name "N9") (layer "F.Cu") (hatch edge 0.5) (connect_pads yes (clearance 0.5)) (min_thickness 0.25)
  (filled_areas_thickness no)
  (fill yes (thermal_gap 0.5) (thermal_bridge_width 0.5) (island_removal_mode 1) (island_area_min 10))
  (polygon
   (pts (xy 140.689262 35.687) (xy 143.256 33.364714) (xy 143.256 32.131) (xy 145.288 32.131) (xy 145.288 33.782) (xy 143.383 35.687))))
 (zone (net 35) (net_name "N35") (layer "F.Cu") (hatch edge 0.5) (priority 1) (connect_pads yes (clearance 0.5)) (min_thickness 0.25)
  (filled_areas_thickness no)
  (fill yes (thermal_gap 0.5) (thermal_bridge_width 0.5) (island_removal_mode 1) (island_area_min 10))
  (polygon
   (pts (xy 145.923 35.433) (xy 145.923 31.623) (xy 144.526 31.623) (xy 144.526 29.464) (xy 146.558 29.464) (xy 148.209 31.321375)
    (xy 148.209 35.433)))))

